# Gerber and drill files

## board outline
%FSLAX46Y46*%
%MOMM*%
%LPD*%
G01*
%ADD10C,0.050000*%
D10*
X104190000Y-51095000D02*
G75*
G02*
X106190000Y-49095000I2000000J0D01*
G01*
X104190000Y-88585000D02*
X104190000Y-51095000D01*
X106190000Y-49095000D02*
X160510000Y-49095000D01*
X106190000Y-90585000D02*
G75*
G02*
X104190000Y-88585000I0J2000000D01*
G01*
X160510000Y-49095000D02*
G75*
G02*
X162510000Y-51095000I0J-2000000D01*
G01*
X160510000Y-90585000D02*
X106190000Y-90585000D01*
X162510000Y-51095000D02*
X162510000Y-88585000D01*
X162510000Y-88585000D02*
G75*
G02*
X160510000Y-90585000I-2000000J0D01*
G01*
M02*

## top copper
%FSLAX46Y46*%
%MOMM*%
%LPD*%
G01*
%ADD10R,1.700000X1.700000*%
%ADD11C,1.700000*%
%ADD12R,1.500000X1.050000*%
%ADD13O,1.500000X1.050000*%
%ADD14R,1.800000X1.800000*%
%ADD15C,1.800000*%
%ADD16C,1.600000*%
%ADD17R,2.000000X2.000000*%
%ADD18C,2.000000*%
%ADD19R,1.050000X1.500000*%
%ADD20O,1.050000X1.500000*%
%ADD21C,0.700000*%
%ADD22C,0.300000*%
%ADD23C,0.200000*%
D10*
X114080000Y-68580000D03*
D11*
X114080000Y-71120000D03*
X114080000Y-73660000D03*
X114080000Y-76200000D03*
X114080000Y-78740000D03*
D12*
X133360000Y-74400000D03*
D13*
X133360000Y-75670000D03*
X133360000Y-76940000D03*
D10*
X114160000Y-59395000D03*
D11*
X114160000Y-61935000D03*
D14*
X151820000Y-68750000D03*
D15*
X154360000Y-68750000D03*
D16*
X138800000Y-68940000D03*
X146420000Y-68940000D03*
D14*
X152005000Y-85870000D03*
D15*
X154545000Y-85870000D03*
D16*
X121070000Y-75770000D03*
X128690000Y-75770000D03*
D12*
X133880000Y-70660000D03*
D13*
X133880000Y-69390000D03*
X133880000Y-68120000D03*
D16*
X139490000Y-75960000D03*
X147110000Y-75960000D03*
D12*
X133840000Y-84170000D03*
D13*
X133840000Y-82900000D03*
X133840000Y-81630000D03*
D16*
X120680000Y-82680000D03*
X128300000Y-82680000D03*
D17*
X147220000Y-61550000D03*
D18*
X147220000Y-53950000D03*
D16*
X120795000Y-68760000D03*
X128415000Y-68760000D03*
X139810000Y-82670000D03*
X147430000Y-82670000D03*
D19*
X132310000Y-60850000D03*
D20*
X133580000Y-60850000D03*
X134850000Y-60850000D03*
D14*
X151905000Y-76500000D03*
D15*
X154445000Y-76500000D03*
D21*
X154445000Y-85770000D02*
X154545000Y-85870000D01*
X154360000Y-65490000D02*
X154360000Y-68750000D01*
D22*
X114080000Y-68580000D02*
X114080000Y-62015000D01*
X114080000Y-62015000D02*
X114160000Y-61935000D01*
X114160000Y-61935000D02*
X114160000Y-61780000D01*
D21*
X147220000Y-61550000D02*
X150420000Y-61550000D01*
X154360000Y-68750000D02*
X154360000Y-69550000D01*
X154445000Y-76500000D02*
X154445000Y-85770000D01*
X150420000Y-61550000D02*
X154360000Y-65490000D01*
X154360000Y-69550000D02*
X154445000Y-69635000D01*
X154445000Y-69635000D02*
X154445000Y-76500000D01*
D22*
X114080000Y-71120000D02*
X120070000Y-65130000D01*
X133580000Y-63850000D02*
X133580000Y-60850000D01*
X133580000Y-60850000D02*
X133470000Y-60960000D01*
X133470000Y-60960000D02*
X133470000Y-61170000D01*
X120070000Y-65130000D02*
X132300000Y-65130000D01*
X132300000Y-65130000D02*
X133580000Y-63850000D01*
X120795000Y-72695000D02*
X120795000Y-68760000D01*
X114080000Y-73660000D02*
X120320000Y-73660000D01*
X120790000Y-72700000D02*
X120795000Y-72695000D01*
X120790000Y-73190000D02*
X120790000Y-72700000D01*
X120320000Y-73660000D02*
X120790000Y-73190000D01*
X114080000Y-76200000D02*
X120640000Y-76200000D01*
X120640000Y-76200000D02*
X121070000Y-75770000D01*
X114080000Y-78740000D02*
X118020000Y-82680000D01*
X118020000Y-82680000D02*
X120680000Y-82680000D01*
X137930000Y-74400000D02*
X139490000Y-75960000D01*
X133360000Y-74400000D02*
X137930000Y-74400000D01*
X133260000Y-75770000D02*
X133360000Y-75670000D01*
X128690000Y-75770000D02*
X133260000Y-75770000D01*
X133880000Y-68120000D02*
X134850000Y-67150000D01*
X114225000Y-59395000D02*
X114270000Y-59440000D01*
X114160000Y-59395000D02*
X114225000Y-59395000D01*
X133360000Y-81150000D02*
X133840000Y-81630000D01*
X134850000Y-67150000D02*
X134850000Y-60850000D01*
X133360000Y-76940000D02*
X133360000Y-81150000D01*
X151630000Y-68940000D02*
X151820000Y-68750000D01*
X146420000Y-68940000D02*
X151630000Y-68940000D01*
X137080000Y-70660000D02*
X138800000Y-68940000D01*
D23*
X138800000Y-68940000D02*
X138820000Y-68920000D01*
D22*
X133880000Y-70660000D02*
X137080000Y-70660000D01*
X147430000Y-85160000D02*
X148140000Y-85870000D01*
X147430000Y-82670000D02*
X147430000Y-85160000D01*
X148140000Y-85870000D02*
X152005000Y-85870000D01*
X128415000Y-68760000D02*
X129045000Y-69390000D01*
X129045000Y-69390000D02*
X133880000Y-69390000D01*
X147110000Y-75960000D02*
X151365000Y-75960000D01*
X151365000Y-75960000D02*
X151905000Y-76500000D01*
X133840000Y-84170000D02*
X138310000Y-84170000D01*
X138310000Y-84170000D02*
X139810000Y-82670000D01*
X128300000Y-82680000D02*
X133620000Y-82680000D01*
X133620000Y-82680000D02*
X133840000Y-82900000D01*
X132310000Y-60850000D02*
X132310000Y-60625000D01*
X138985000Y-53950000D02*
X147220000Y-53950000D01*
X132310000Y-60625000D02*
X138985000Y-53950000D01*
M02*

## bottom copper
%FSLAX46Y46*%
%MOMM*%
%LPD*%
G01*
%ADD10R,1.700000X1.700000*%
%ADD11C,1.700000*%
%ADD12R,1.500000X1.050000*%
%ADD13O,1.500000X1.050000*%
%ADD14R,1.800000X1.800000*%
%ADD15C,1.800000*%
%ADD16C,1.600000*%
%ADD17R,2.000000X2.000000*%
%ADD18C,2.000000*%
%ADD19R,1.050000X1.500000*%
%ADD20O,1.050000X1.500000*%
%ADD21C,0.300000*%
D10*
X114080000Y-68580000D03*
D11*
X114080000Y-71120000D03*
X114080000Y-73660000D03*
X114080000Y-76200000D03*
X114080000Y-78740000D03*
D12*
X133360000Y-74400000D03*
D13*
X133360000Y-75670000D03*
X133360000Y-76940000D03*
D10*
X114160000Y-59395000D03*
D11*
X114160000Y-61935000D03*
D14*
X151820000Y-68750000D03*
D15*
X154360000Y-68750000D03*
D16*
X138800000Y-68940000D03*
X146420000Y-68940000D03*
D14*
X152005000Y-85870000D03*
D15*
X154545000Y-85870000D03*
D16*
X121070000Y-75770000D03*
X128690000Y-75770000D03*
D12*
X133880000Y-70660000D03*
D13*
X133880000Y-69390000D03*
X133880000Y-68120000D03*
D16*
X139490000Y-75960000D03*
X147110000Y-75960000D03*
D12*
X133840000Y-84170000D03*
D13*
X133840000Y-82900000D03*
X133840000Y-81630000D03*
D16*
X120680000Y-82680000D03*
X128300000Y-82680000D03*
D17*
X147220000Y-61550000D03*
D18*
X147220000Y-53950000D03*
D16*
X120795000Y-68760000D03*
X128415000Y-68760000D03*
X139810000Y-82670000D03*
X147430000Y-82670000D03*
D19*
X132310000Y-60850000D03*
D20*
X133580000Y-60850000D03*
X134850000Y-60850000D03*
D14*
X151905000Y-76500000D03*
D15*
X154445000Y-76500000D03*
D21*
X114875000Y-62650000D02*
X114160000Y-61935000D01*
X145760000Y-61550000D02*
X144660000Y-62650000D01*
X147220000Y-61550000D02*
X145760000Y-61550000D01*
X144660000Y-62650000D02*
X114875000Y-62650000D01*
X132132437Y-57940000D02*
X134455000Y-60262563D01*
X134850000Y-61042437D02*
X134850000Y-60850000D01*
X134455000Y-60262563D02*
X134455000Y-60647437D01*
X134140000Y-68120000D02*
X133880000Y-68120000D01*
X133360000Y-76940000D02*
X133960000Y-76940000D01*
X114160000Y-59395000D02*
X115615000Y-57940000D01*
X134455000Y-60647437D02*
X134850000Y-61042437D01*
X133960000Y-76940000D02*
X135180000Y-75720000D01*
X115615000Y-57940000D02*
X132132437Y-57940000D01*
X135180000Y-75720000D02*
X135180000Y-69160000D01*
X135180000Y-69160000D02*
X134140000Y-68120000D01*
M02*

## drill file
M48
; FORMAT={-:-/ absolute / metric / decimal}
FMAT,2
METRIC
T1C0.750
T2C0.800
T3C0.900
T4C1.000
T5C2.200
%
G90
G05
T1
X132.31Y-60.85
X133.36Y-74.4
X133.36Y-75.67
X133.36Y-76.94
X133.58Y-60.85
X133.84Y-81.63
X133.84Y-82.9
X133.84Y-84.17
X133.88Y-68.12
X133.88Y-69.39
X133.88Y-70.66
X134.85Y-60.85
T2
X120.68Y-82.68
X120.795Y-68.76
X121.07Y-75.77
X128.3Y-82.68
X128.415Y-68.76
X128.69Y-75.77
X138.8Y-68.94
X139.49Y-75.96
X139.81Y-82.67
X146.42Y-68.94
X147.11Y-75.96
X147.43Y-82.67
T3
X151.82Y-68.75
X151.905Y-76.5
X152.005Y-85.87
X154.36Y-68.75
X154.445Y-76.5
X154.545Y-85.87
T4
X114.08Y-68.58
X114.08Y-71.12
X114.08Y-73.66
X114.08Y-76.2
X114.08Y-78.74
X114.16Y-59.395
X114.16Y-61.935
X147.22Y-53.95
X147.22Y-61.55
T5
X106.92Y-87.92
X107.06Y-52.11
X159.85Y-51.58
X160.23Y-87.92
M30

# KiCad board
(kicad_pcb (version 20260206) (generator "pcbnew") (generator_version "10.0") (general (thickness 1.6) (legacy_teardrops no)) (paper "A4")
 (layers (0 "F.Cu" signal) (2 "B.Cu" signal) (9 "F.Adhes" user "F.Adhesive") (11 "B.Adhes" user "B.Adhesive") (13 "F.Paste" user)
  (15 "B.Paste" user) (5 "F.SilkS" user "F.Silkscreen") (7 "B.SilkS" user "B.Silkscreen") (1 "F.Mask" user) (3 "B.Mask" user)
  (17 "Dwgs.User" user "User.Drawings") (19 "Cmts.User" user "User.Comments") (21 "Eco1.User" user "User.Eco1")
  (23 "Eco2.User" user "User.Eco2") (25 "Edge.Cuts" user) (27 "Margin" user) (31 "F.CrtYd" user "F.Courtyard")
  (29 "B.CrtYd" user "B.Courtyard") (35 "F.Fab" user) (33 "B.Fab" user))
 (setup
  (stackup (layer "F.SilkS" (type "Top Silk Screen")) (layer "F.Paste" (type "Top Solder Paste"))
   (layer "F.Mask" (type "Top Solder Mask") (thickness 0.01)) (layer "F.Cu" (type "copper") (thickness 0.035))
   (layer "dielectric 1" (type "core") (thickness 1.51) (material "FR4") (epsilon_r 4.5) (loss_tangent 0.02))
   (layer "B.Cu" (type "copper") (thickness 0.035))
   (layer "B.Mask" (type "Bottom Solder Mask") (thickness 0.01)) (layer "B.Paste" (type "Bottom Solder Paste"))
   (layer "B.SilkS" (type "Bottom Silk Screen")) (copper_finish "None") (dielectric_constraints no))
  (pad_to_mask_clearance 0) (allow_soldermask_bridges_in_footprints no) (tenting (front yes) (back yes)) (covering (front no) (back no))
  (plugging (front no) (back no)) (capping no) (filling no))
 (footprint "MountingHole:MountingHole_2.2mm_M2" (layer "F.Cu") (at 106.92 87.92)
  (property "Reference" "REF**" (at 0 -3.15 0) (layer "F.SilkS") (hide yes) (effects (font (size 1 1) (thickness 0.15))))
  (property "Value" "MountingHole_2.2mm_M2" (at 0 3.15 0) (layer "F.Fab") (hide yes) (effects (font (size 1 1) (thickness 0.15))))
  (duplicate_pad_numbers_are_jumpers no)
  (pad "" np_thru_hole circle (at 0 0) (size 2.2 2.2) (drill 2.2) (layers "*.Cu" "*.Mask")))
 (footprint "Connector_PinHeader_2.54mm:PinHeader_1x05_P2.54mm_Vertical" (layer "F.Cu") (at 114.08 68.58)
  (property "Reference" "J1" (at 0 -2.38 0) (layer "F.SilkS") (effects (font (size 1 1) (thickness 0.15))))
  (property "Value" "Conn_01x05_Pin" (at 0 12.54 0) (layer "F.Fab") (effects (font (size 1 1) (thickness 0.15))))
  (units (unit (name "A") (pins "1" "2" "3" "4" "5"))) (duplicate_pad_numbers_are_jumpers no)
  (pad "1" thru_hole rect (at 0 0) (size 1.7 1.7) (drill 1) (layers "*.Cu" "*.Mask") (remove_unused_layers no) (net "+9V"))
  (pad "2" thru_hole circle (at 0 2.54) (size 1.7 1.7) (drill 1) (layers "*.Cu" "*.Mask") (remove_unused_layers no) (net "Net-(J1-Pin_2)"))
  (pad "3" thru_hole circle (at 0 5.08) (size 1.7 1.7) (drill 1) (layers "*.Cu" "*.Mask") (remove_unused_layers no) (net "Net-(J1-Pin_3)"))
  (pad "4" thru_hole circle (at 0 7.62) (size 1.7 1.7) (drill 1) (layers "*.Cu" "*.Mask") (remove_unused_layers no) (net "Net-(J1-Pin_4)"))
  (pad "5" thru_hole circle (at 0 10.16) (size 1.7 1.7) (drill 1) (layers "*.Cu" "*.Mask") (remove_unused_layers no) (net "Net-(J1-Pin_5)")))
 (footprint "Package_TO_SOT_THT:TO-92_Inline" (layer "F.Cu") (at 133.36 74.4 -90)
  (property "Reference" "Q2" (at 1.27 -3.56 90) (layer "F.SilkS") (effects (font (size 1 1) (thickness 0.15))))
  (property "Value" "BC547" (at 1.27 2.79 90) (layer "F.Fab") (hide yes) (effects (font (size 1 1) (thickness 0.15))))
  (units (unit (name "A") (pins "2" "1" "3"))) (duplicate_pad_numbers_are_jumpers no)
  (pad "1" thru_hole rect (at 0 0 270) (size 1.05 1.5) (drill 0.75) (layers "*.Cu" "*.Mask") (remove_unused_layers no) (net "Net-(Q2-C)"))
  (pad "2" thru_hole oval (at 1.27 0 270) (size 1.05 1.5) (drill 0.75) (layers "*.Cu" "*.Mask") (remove_unused_layers no) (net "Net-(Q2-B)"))
  (pad "3" thru_hole oval (at 2.54 0 270) (size 1.05 1.5) (drill 0.75) (layers "*.Cu" "*.Mask") (remove_unused_layers no) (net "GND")))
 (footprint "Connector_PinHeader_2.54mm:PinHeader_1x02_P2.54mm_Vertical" (layer "F.Cu") (at 114.16 59.395)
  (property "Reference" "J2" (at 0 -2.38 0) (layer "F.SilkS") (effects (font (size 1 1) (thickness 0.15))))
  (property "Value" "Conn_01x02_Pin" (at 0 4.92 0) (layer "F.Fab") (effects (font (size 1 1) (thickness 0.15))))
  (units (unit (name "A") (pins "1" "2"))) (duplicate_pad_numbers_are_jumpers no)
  (pad "1" thru_hole rect (at 0 0) (size 1.7 1.7) (drill 1) (layers "*.Cu" "*.Mask") (remove_unused_layers no) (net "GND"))
  (pad "2" thru_hole circle (at 0 2.54) (size 1.7 1.7) (drill 1) (layers "*.Cu" "*.Mask") (remove_unused_layers no) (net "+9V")))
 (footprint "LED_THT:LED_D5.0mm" (layer "F.Cu") (at 151.82 68.75)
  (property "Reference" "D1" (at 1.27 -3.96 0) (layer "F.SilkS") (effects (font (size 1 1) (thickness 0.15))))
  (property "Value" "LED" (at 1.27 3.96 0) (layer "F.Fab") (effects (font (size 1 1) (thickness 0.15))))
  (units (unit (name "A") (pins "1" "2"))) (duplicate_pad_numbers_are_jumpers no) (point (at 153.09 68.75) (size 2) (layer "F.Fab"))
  (pad "1" thru_hole rect (at 0 0) (size 1.8 1.8) (drill 0.9) (layers "*.Cu" "*.Mask") (remove_unused_layers no) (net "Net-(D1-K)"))
  (pad "2" thru_hole circle (at 2.54 0) (size 1.8 1.8) (drill 0.9) (layers "*.Cu" "*.Mask") (remove_unused_layers no) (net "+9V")))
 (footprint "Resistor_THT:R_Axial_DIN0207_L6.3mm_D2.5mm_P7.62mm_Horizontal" (layer "F.Cu") (at 138.8 68.94)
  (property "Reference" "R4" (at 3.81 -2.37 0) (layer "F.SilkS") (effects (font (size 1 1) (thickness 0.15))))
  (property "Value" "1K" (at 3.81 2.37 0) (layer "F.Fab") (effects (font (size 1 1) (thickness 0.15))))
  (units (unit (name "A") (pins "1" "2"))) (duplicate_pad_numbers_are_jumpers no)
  (pad "1" thru_hole circle (at 0 0) (size 1.6 1.6) (drill 0.8) (layers "*.Cu" "*.Mask") (remove_unused_layers no) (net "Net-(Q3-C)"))
  (pad "2" thru_hole circle (at 7.62 0) (size 1.6 1.6) (drill 0.8) (layers "*.Cu" "*.Mask") (remove_unused_layers no) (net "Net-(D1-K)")))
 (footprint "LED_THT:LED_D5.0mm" (layer "F.Cu") (at 152.005 85.87)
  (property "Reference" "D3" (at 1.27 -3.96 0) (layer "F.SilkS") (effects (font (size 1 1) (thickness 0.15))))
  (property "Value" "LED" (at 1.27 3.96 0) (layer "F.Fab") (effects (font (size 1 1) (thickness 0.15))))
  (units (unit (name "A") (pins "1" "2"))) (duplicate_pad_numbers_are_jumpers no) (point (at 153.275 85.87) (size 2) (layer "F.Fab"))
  (pad "1" thru_hole rect (at 0 0) (size 1.8 1.8) (drill 0.9) (layers "*.Cu" "*.Mask") (remove_unused_layers no) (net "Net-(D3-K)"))
  (pad "2" thru_hole circle (at 2.54 0) (size 1.8 1.8) (drill 0.9) (layers "*.Cu" "*.Mask") (remove_unused_layers no) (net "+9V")))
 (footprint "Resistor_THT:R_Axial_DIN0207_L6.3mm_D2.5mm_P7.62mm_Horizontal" (layer "F.Cu") (at 121.07 75.77)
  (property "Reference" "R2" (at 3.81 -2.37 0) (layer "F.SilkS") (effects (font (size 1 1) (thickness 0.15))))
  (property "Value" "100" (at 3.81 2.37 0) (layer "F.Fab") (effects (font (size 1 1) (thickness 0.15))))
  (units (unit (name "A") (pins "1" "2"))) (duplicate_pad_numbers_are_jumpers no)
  (pad "1" thru_hole circle (at 0 0) (size 1.6 1.6) (drill 0.8) (layers "*.Cu" "*.Mask") (remove_unused_layers no) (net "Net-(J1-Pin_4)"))
  (pad "2" thru_hole circle (at 7.62 0) (size 1.6 1.6) (drill 0.8) (layers "*.Cu" "*.Mask") (remove_unused_layers no) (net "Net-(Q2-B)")))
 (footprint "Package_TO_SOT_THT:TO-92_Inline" (layer "F.Cu") (at 133.88 70.66 90)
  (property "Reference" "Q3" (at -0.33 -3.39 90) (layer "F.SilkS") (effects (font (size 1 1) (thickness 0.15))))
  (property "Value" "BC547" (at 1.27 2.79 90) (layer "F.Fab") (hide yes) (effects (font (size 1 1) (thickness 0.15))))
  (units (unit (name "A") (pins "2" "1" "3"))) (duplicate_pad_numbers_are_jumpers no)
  (pad "1" thru_hole rect (at 0 0 90) (size 1.05 1.5) (drill 0.75) (layers "*.Cu" "*.Mask") (remove_unused_layers no) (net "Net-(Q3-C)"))
  (pad "2" thru_hole oval (at 1.27 0 90) (size 1.05 1.5) (drill 0.75) (layers "*.Cu" "*.Mask") (remove_unused_layers no) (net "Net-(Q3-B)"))
  (pad "3" thru_hole oval (at 2.54 0 90) (size 1.05 1.5) (drill 0.75) (layers "*.Cu" "*.Mask") (remove_unused_layers no) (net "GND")))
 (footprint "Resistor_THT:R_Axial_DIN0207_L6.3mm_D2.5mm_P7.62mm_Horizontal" (layer "F.Cu") (at 139.49 75.96)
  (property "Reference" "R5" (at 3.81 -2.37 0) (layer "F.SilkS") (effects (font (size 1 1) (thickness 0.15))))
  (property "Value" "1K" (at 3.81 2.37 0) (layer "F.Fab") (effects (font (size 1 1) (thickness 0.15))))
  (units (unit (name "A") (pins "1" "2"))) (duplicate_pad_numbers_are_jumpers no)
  (pad "1" thru_hole circle (at 0 0) (size 1.6 1.6) (drill 0.8) (layers "*.Cu" "*.Mask") (remove_unused_layers no) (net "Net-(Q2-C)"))
  (pad "2" thru_hole circle (at 7.62 0) (size 1.6 1.6) (drill 0.8) (layers "*.Cu" "*.Mask") (remove_unused_layers no) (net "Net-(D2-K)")))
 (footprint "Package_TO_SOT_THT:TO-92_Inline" (layer "F.Cu") (at 133.84 84.17 90)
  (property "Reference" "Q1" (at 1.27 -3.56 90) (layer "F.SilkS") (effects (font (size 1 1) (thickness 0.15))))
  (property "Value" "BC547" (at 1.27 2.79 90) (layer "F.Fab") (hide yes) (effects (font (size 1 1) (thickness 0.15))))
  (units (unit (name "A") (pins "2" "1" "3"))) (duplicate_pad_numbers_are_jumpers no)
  (pad "1" thru_hole rect (at 0 0 90) (size 1.05 1.5) (drill 0.75) (layers "*.Cu" "*.Mask") (remove_unused_layers no) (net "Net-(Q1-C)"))
  (pad "2" thru_hole oval (at 1.27 0 90) (size 1.05 1.5) (drill 0.75) (layers "*.Cu" "*.Mask") (remove_unused_layers no) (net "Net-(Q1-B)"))
  (pad "3" thru_hole oval (at 2.54 0 90) (size 1.05 1.5) (drill 0.75) (layers "*.Cu" "*.Mask") (remove_unused_layers no) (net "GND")))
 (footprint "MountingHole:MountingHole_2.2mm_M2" (layer "F.Cu") (at 160.23 87.92)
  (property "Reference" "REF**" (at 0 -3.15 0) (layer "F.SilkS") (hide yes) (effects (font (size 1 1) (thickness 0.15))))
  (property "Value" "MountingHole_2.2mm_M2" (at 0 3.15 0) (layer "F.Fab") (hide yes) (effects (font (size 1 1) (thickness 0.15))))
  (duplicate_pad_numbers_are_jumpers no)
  (pad "" np_thru_hole circle (at 0 0) (size 2.2 2.2) (drill 2.2) (layers "*.Cu" "*.Mask")))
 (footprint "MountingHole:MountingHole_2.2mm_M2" (layer "F.Cu") (at 159.85 51.58)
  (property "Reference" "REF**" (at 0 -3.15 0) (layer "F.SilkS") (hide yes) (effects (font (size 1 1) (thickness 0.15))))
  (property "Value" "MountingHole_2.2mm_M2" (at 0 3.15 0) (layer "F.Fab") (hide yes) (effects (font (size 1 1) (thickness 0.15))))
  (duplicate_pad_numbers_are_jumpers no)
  (pad "" np_thru_hole circle (at 0 0) (size 2.2 2.2) (drill 2.2) (layers "*.Cu" "*.Mask")))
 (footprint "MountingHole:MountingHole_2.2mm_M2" (layer "F.Cu") (at 107.06 52.11)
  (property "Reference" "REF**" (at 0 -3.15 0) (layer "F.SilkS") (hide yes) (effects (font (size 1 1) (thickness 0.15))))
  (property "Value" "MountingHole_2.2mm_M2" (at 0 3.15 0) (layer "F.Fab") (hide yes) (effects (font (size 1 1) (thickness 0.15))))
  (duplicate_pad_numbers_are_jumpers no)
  (pad "" np_thru_hole circle (at 0 0) (size 2.2 2.2) (drill 2.2) (layers "*.Cu" "*.Mask")))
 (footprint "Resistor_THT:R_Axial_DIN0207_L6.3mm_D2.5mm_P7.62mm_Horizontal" (layer "F.Cu") (at 120.68 82.68)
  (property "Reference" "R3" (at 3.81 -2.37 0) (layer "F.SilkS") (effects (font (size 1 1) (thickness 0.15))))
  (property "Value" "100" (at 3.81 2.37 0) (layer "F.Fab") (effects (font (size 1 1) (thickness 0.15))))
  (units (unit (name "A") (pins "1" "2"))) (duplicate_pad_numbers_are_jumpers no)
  (pad "1" thru_hole circle (at 0 0) (size 1.6 1.6) (drill 0.8) (layers "*.Cu" "*.Mask") (remove_unused_layers no) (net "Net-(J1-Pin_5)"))
  (pad "2" thru_hole circle (at 7.62 0) (size 1.6 1.6) (drill 0.8) (layers "*.Cu" "*.Mask") (remove_unused_layers no) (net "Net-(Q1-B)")))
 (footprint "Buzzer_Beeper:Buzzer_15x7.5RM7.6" (layer "F.Cu") (at 147.22 61.55 90)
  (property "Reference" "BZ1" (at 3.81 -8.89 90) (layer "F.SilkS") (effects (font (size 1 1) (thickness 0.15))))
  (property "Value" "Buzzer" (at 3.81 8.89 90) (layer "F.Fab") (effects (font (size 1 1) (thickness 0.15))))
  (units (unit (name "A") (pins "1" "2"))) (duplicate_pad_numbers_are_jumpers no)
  (pad "1" thru_hole rect (at 0 0 90) (size 2 2) (drill 1) (layers "*.Cu" "*.Mask") (remove_unused_layers no) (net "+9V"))
  (pad "2" thru_hole circle (at 7.6 0 90) (size 2 2) (drill 1) (layers "*.Cu" "*.Mask") (remove_unused_layers no) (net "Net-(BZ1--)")))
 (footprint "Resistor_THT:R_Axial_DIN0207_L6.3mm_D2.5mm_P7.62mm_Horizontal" (layer "F.Cu") (at 120.795 68.76)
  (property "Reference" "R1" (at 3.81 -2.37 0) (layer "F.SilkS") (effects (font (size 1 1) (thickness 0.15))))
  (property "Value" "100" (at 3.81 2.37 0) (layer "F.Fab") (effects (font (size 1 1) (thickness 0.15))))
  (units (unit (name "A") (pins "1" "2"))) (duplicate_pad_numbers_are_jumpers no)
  (pad "1" thru_hole circle (at 0 0) (size 1.6 1.6) (drill 0.8) (layers "*.Cu" "*.Mask") (remove_unused_layers no) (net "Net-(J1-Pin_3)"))
  (pad "2" thru_hole circle (at 7.62 0) (size 1.6 1.6) (drill 0.8) (layers "*.Cu" "*.Mask") (remove_unused_layers no) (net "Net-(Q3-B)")))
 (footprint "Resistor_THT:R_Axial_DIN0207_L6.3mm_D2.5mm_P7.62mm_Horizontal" (layer "F.Cu") (at 139.81 82.67)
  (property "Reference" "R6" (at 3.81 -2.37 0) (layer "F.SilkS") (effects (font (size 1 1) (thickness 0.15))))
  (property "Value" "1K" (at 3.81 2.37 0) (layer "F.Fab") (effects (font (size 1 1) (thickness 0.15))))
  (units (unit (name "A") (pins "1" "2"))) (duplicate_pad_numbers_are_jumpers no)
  (pad "1" thru_hole circle (at 0 0) (size 1.6 1.6) (drill 0.8) (layers "*.Cu" "*.Mask") (remove_unused_layers no) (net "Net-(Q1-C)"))
  (pad "2" thru_hole circle (at 7.62 0) (size 1.6 1.6) (drill 0.8) (layers "*.Cu" "*.Mask") (remove_unused_layers no) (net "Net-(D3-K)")))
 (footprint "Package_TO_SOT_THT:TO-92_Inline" (layer "F.Cu") (at 132.31 60.85)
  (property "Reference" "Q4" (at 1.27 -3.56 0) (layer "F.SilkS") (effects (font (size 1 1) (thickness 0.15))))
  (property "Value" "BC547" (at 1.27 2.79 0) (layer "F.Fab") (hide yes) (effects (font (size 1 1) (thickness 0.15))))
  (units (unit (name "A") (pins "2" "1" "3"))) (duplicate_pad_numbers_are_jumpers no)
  (pad "1" thru_hole rect (at 0 0) (size 1.05 1.5) (drill 0.75) (layers "*.Cu" "*.Mask") (remove_unused_layers no) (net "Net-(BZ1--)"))
  (pad "2" thru_hole oval (at 1.27 0) (size 1.05 1.5) (drill 0.75) (layers "*.Cu" "*.Mask") (remove_unused_layers no) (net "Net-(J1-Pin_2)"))
  (pad "3" thru_hole oval (at 2.54 0) (size 1.05 1.5) (drill 0.75) (layers "*.Cu" "*.Mask") (remove_unused_layers no) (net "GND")))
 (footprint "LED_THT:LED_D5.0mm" (layer "F.Cu") (at 151.905 76.5)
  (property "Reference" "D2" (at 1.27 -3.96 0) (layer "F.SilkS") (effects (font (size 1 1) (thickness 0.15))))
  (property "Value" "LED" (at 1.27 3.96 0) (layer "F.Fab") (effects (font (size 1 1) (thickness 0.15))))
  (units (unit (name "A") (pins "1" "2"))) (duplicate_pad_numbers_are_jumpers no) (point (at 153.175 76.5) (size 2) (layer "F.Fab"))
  (pad "1" thru_hole rect (at 0 0) (size 1.8 1.8) (drill 0.9) (layers "*.Cu" "*.Mask") (remove_unused_layers no) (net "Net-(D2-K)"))
  (pad "2" thru_hole circle (at 2.54 0) (size 1.8 1.8) (drill 0.9) (layers "*.Cu" "*.Mask") (remove_unused_layers no) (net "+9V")))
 (gr_arc (start 104.19 51.095) (mid 104.775786 49.680786) (end 106.19 49.095) (stroke (width 0.05) (type default)) (layer "Edge.Cuts"))
 (gr_line (start 104.19 88.585) (end 104.19 51.095) (stroke (width 0.05) (type default)) (layer "Edge.Cuts"))
 (gr_line (start 106.19 49.095) (end 160.51 49.095) (stroke (width 0.05) (type default)) (layer "Edge.Cuts"))
 (gr_arc (start 106.19 90.585) (mid 104.775786 89.999214) (end 104.19 88.585) (stroke (width 0.05) (type default)) (layer "Edge.Cuts"))
 (gr_arc (start 160.51 49.095) (mid 161.924214 49.680786) (end 162.51 51.095) (stroke (width 0.05) (type default)) (layer "Edge.Cuts"))
 (gr_line (start 160.51 90.585) (end 106.19 90.585) (stroke (width 0.05) (type default)) (layer "Edge.Cuts"))
 (gr_line (start 162.51 51.095) (end 162.51 88.585) (stroke (width 0.05) (type default)) (layer "Edge.Cuts"))
 (gr_arc (start 162.51 88.585) (mid 161.924214 89.999214) (end 160.51 90.585) (stroke (width 0.05) (type default)) (layer "Edge.Cuts"))
 (segment (start 154.445 85.77) (end 154.545 85.87) (width 0.7) (layer "F.Cu") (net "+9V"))
 (segment (start 154.36 65.49) (end 154.36 68.75) (width 0.7) (layer "F.Cu") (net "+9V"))
 (segment (start 114.08 68.58) (end 114.08 62.015) (width 0.3) (layer "F.Cu") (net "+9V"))
 (segment (start 114.08 62.015) (end 114.16 61.935) (width 0.3) (layer "F.Cu") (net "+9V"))
 (segment (start 114.16 61.935) (end 114.16 61.78) (width 0.3) (layer "F.Cu") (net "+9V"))
 (segment (start 147.22 61.55) (end 150.42 61.55) (width 0.7) (layer "F.Cu") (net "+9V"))
 (segment (start 154.36 68.75) (end 154.36 69.55) (width 0.7) (layer "F.Cu") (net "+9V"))
 (segment (start 154.445 76.5) (end 154.445 85.77) (width 0.7) (layer "F.Cu") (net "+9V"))
 (segment (start 150.42 61.55) (end 154.36 65.49) (width 0.7) (layer "F.Cu") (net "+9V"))
 (segment (start 154.36 69.55) (end 154.445 69.635) (width 0.7) (layer "F.Cu") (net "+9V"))
 (segment (start 154.445 69.635) (end 154.445 76.5) (width 0.7) (layer "F.Cu") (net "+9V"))
 (segment (start 114.875 62.65) (end 114.16 61.935) (width 0.3) (layer "B.Cu") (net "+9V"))
 (segment (start 145.76 61.55) (end 144.66 62.65) (width 0.3) (layer "B.Cu") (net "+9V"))
 (segment (start 147.22 61.55) (end 145.76 61.55) (width 0.3) (layer "B.Cu") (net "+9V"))
 (segment (start 144.66 62.65) (end 114.875 62.65) (width 0.3) (layer "B.Cu") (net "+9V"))
 (segment (start 114.08 71.12) (end 120.07 65.13) (width 0.3) (layer "F.Cu") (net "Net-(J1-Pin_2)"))
 (segment (start 133.58 63.85) (end 133.58 60.85) (width 0.3) (layer "F.Cu") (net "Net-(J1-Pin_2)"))
 (segment (start 133.58 60.85) (end 133.47 60.96) (width 0.3) (layer "F.Cu") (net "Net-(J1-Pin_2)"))
 (segment (start 133.47 60.96) (end 133.47 61.17) (width 0.3) (layer "F.Cu") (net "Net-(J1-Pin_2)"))
 (segment (start 120.07 65.13) (end 132.3 65.13) (width 0.3) (layer "F.Cu") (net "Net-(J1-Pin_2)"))
 (segment (start 132.3 65.13) (end 133.58 63.85) (width 0.3) (layer "F.Cu") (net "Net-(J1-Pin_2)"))
 (segment (start 120.795 72.695) (end 120.795 68.76) (width 0.3) (layer "F.Cu") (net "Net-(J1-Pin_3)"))
 (segment (start 114.08 73.66) (end 120.32 73.66) (width 0.3) (layer "F.Cu") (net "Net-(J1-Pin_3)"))
 (segment (start 120.79 72.7) (end 120.795 72.695) (width 0.3) (layer "F.Cu") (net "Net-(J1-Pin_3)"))
 (segment (start 120.79 73.19) (end 120.79 72.7) (width 0.3) (layer "F.Cu") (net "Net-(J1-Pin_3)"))
 (segment (start 120.32 73.66) (end 120.79 73.19) (width 0.3) (layer "F.Cu") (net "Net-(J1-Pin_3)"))
 (segment (start 114.08 76.2) (end 120.64 76.2) (width 0.3) (layer "F.Cu") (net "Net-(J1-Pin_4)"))
 (segment (start 120.64 76.2) (end 121.07 75.77) (width 0.3) (layer "F.Cu") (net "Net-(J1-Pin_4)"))
 (segment (start 114.08 78.74) (end 118.02 82.68) (width 0.3) (layer "F.Cu") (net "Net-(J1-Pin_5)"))
 (segment (start 118.02 82.68) (end 120.68 82.68) (width 0.3) (layer "F.Cu") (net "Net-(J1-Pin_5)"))
 (segment (start 137.93 74.4) (end 139.49 75.96) (width 0.3) (layer "F.Cu") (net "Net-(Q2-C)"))
 (segment (start 133.36 74.4) (end 137.93 74.4) (width 0.3) (layer "F.Cu") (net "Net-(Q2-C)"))
 (segment (start 133.26 75.77) (end 133.36 75.67) (width 0.3) (layer "F.Cu") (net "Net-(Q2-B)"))
 (segment (start 128.69 75.77) (end 133.26 75.77) (width 0.3) (layer "F.Cu") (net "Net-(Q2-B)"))
 (segment (start 133.88 68.12) (end 134.85 67.15) (width 0.3) (layer "F.Cu") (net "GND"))
 (segment (start 114.225 59.395) (end 114.27 59.44) (width 0.3) (layer "F.Cu") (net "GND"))
 (segment (start 114.16 59.395) (end 114.225 59.395) (width 0.3) (layer "F.Cu") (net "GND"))
 (segment (start 133.36 81.15) (end 133.84 81.63) (width 0.3) (layer "F.Cu") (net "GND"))
 (segment (start 134.85 67.15) (end 134.85 60.85) (width 0.3) (layer "F.Cu") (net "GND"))
 (segment (start 133.36 76.94) (end 133.36 81.15) (width 0.3) (layer "F.Cu") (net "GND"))
 (segment (start 132.132437 57.94) (end 134.455 60.262563) (width 0.3) (layer "B.Cu") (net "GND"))
 (segment (start 134.85 61.042437) (end 134.85 60.85) (width 0.3) (layer "B.Cu") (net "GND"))
 (segment (start 134.455 60.262563) (end 134.455 60.647437) (width 0.3) (layer "B.Cu") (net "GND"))
 (segment (start 134.14 68.12) (end 133.88 68.12) (width 0.3) (layer "B.Cu") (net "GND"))
 (segment (start 133.36 76.94) (end 133.96 76.94) (width 0.3) (layer "B.Cu") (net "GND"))
 (segment (start 114.16 59.395) (end 115.615 57.94) (width 0.3) (layer "B.Cu") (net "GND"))
 (segment (start 134.455 60.647437) (end 134.85 61.042437) (width 0.3) (layer "B.Cu") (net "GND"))
 (segment (start 133.96 76.94) (end 135.18 75.72) (width 0.3) (layer "B.Cu") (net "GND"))
 (segment (start 115.615 57.94) (end 132.132437 57.94) (width 0.3) (layer "B.Cu") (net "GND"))
 (segment (start 135.18 75.72) (end 135.18 69.16) (width 0.3) (layer "B.Cu") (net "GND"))
 (segment (start 135.18 69.16) (end 134.14 68.12) (width 0.3) (layer "B.Cu") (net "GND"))
 (segment (start 151.63 68.94) (end 151.82 68.75) (width 0.3) (layer "F.Cu") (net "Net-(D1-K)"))
 (segment (start 146.42 68.94) (end 151.63 68.94) (width 0.3) (layer "F.Cu") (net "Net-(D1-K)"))
 (segment (start 137.08 70.66) (end 138.8 68.94) (width 0.3) (layer "F.Cu") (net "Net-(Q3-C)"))
 (segment (start 138.8 68.94) (end 138.82 68.92) (width 0.2) (layer "F.Cu") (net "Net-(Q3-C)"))
 (segment (start 133.88 70.66) (end 137.08 70.66) (width 0.3) (layer "F.Cu") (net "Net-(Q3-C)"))
 (segment (start 147.43 85.16) (end 148.14 85.87) (width 0.3) (layer "F.Cu") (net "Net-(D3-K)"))
 (segment (start 147.43 82.67) (end 147.43 85.16) (width 0.3) (layer "F.Cu") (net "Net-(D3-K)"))
 (segment (start 148.14 85.87) (end 152.005 85.87) (width 0.3) (layer "F.Cu") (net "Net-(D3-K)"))
 (segment (start 128.415 68.76) (end 129.045 69.39) (width 0.3) (layer "F.Cu") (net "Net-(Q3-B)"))
 (segment (start 129.045 69.39) (end 133.88 69.39) (width 0.3) (layer "F.Cu") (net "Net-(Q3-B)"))
 (segment (start 147.11 75.96) (end 151.365 75.96) (width 0.3) (layer "F.Cu") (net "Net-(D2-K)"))
 (segment (start 151.365 75.96) (end 151.905 76.5) (width 0.3) (layer "F.Cu") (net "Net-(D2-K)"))
 (segment (start 133.84 84.17) (end 138.31 84.17) (width 0.3) (layer "F.Cu") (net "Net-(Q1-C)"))
 (segment (start 138.31 84.17) (end 139.81 82.67) (width 0.3) (layer "F.Cu") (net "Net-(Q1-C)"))
 (segment (start 128.3 82.68) (end 133.62 82.68) (width 0.3) (layer "F.Cu") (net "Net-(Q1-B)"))
 (segment (start 133.62 82.68) (end 133.84 82.9) (width 0.3) (layer "F.Cu") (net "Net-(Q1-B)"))
 (segment (start 132.31 60.85) (end 132.31 60.625) (width 0.3) (layer "F.Cu") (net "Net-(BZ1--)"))
 (segment (start 138.985 53.95) (end 147.22 53.95) (width 0.3) (layer "F.Cu") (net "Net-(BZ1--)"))
 (segment (start 132.31 60.625) (end 138.985 53.95) (width 0.3) (layer "F.Cu") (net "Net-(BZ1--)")))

